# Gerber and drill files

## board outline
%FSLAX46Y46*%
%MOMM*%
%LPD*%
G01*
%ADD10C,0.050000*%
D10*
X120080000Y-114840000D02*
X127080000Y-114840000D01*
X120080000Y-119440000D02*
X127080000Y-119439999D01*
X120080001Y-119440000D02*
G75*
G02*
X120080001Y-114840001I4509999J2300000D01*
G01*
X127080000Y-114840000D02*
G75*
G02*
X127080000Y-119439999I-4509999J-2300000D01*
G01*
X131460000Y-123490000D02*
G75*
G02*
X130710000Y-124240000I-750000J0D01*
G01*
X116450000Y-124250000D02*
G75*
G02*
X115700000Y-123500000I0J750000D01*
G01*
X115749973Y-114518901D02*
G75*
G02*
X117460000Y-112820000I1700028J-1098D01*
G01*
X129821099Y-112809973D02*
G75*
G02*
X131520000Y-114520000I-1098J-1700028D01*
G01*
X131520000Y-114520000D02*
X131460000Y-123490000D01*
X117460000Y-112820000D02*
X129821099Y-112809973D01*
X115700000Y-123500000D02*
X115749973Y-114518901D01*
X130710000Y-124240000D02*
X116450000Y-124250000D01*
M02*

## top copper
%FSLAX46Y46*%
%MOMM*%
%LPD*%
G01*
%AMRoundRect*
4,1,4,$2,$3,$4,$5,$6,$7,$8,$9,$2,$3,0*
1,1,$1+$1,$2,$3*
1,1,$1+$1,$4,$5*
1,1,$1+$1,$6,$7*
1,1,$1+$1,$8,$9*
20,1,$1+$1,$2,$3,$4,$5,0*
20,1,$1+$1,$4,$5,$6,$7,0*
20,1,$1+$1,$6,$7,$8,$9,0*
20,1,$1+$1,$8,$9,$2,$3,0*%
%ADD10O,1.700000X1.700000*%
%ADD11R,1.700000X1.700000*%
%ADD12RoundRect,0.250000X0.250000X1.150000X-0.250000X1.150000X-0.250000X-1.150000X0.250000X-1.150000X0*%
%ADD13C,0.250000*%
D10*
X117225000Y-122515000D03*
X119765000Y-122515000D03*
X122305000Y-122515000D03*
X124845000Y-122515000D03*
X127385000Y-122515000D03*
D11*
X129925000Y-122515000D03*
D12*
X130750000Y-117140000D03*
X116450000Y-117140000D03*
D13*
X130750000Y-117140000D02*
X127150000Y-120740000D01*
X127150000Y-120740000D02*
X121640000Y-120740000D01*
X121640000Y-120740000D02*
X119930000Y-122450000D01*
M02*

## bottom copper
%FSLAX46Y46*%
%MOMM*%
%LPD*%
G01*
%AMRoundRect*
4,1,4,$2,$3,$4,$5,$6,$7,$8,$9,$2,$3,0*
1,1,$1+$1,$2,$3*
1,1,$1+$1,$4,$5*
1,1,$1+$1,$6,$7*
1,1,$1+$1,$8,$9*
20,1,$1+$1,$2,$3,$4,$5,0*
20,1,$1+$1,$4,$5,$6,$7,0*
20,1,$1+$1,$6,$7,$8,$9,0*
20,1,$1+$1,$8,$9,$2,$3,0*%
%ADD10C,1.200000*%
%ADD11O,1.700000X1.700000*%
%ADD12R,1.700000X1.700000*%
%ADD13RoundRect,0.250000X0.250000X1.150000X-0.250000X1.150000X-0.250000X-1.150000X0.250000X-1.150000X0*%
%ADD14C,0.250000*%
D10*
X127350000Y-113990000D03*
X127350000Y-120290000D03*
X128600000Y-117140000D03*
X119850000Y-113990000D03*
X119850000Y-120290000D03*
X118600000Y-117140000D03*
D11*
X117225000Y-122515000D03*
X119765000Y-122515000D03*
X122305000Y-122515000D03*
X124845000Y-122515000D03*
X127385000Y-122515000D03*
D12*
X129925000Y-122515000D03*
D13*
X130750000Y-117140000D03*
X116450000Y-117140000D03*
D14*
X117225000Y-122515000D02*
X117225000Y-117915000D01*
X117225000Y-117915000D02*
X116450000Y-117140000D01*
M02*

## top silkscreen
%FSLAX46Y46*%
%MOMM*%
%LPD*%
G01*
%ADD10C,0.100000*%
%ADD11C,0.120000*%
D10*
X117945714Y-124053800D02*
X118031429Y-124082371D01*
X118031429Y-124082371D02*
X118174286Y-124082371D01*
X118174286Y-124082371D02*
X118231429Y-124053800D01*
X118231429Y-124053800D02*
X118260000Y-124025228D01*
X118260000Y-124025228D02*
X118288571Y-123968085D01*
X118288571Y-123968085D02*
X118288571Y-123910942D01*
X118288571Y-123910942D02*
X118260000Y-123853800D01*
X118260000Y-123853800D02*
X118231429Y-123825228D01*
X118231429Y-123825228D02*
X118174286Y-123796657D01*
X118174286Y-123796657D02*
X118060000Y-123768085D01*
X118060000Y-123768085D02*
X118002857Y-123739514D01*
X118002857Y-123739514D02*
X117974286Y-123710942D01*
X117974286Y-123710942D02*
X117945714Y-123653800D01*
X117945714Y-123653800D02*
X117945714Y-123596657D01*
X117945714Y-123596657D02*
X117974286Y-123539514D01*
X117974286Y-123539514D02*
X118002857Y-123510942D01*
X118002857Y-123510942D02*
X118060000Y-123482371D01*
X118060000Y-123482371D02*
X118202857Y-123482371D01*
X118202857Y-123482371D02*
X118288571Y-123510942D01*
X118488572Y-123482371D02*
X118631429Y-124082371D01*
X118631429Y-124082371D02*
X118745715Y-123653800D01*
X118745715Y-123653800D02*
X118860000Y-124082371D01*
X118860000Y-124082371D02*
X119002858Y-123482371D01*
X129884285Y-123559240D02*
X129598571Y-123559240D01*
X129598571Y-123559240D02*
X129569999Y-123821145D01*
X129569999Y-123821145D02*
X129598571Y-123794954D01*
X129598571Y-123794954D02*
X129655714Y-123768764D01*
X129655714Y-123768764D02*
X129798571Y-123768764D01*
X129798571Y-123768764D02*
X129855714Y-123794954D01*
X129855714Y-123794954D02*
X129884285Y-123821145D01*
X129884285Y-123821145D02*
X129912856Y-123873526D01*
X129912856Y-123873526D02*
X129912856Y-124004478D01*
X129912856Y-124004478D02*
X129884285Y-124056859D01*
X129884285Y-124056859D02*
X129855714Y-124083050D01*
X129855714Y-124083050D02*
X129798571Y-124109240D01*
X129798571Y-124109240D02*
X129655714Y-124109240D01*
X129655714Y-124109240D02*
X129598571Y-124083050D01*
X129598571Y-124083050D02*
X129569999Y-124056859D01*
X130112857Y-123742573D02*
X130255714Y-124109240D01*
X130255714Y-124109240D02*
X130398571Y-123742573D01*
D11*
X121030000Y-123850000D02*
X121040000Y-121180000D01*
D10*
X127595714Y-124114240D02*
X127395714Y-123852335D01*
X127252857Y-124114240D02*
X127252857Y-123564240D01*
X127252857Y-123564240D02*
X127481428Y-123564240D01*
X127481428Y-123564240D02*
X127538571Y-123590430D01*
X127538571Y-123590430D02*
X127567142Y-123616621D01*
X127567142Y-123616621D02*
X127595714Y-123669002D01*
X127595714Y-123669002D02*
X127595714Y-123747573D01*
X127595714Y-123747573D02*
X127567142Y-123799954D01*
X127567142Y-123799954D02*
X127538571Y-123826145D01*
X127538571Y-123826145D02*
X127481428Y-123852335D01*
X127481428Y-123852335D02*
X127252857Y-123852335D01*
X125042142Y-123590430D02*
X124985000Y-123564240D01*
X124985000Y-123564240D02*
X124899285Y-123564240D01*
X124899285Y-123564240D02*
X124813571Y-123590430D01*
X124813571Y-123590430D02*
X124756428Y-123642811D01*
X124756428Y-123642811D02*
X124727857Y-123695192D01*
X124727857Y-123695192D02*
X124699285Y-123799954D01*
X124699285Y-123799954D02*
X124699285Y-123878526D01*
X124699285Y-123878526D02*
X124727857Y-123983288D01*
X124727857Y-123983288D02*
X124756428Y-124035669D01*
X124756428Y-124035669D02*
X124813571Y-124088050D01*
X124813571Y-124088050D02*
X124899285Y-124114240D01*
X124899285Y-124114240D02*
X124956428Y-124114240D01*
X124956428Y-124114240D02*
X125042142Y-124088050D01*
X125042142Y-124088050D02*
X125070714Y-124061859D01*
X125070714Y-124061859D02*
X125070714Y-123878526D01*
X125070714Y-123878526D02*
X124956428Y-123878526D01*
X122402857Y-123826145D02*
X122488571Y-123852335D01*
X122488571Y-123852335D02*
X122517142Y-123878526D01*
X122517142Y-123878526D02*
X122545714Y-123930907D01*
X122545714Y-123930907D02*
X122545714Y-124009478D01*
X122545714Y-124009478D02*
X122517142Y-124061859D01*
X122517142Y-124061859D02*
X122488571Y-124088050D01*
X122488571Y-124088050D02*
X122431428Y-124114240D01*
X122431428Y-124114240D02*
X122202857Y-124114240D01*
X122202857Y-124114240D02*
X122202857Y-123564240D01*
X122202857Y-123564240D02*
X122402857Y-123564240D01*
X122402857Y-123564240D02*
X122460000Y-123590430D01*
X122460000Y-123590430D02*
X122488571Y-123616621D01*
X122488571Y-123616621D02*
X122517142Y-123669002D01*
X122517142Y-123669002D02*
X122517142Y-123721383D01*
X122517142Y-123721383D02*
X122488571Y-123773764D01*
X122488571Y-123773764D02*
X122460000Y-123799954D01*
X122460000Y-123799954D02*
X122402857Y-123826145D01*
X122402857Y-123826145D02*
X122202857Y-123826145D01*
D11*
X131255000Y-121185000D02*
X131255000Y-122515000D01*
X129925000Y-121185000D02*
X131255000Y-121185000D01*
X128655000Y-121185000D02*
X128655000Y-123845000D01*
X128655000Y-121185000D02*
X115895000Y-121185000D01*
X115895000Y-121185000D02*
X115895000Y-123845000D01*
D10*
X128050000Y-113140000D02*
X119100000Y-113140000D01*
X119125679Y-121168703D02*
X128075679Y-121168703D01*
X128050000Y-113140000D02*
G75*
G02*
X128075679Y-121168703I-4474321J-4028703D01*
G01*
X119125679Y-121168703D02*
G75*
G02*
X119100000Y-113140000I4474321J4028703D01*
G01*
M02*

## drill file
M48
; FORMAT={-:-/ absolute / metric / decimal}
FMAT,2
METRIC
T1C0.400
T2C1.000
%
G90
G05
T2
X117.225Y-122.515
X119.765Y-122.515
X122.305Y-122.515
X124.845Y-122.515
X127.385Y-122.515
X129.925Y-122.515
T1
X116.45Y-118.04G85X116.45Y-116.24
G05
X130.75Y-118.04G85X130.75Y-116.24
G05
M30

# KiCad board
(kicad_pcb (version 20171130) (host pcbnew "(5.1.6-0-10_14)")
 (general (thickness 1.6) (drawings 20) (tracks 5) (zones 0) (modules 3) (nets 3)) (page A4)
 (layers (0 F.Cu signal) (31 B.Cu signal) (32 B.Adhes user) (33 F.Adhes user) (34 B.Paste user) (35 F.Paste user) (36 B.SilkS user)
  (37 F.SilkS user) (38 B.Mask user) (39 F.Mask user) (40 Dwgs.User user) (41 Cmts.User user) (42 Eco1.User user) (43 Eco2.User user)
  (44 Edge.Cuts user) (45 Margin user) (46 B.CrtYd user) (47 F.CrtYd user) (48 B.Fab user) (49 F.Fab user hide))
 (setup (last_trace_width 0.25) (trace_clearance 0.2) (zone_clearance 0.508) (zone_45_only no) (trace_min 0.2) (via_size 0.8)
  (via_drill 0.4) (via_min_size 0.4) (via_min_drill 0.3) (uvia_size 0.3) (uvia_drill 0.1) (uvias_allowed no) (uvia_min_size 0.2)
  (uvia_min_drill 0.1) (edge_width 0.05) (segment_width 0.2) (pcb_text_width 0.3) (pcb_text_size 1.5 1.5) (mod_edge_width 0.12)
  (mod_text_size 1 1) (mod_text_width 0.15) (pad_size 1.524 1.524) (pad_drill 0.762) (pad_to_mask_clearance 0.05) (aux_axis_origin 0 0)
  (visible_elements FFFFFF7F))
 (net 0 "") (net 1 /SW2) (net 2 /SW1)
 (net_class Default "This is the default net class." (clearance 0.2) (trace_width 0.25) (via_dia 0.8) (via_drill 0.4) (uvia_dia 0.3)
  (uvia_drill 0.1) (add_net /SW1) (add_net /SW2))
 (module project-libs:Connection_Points (layer B.Cu) (at 123.6 117.14)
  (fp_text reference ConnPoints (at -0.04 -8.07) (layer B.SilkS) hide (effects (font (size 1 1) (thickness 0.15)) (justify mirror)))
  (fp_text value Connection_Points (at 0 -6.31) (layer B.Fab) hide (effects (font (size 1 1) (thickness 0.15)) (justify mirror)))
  (pad "" smd circle (at 3.75 -3.15) (size 1.2 1.2) (layers B.Cu B.Paste B.Mask))
  (pad "" smd circle (at 3.75 3.15) (size 1.2 1.2) (layers B.Cu B.Paste B.Mask))
  (pad "" smd circle (at 5 0) (size 1.2 1.2) (layers B.Cu B.Paste B.Mask))
  (pad "" smd circle (at -3.75 -3.15) (size 1.2 1.2) (layers B.Cu B.Paste B.Mask))
  (pad "" smd circle (at -3.75 3.15) (size 1.2 1.2) (layers B.Cu B.Paste B.Mask))
  (pad "" smd circle (at -5 0) (size 1.2 1.2) (layers B.Cu B.Paste B.Mask)))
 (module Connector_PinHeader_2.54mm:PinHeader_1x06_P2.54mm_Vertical (layer F.Cu) (at 129.925 122.515 270)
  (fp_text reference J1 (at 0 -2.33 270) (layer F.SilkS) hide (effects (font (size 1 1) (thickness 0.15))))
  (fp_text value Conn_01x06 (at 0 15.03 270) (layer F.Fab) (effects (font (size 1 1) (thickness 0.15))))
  (fp_line (start -1.33 -1.33) (end 0 -1.33) (layer F.SilkS) (width 0.12))
  (fp_line (start -1.33 0) (end -1.33 -1.33) (layer F.SilkS) (width 0.12))
  (fp_line (start -1.33 1.27) (end 1.33 1.27) (layer F.SilkS) (width 0.12))
  (fp_line (start -1.33 1.27) (end -1.33 14.03) (layer F.SilkS) (width 0.12))
  (fp_line (start -1.33 14.03) (end 1.33 14.03) (layer F.SilkS) (width 0.12))
  (pad 6 thru_hole oval (at 0 12.7 270) (size 1.7 1.7) (drill 1) (layers *.Cu *.Mask) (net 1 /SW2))
  (pad 5 thru_hole oval (at 0 10.16 270) (size 1.7 1.7) (drill 1) (layers *.Cu *.Mask) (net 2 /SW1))
  (pad 4 thru_hole oval (at 0 7.62 270) (size 1.7 1.7) (drill 1) (layers *.Cu *.Mask))
  (pad 3 thru_hole oval (at 0 5.08 270) (size 1.7 1.7) (drill 1) (layers *.Cu *.Mask))
  (pad 2 thru_hole oval (at 0 2.54 270) (size 1.7 1.7) (drill 1) (layers *.Cu *.Mask))
  (pad 1 thru_hole rect (at 0 0 270) (size 1.7 1.7) (drill 1) (layers *.Cu *.Mask)))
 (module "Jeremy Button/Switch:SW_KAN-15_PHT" (layer F.Cu) (at 123.6 117.14 180)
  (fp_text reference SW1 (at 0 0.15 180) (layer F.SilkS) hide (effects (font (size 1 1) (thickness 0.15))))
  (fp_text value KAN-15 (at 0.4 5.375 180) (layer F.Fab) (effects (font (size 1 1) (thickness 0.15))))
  (fp_line (start -4.45 4) (end 4.5 4) (layer F.SilkS) (width 0.1))
  (fp_line (start 4.474321 -4.028703) (end -4.475679 -4.028703) (layer F.SilkS) (width 0.1))
  (fp_arc (start 0.024321 -0.028703) (end -4.475679 -4.028703) (angle -83.63358372) (layer F.SilkS) (width 0.1))
  (fp_arc (start 0 0) (end 4.5 4) (angle -83.63358372) (layer F.SilkS) (width 0.1))
  (pad 1 thru_hole roundrect (at -7.15 0 180) (size 1 2.8) (drill oval 0.4 2.2) (layers *.Cu *.Mask) (roundrect_rratio 0.25) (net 2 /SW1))
  (pad 2 thru_hole roundrect (at 7.15 0 180) (size 1 2.8) (drill oval 0.4 2.2) (layers *.Cu *.Mask) (roundrect_rratio 0.25) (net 1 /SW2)))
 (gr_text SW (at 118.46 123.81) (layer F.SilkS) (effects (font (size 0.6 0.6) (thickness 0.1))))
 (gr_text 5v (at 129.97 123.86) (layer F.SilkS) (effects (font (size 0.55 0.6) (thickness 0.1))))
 (gr_line (start 121.03 123.85) (end 121.04 121.18) (layer F.SilkS) (width 0.12))
 (gr_line (start 120.08 114.84) (end 127.08 114.84) (layer Edge.Cuts) (width 0.05))
 (gr_line (start 120.08 119.44) (end 127.08 119.439999) (layer Edge.Cuts) (width 0.05))
 (gr_arc (start 124.59 117.14) (end 120.080001 114.840001) (angle -54.04114679) (layer Edge.Cuts) (width 0.05))
 (gr_arc (start 122.570001 117.14) (end 127.08 119.439999) (angle -54.04114679) (layer Edge.Cuts) (width 0.05))
 (gr_arc (start 130.71 123.49) (end 130.71 124.24) (angle -90) (layer Edge.Cuts) (width 0.05))
 (gr_arc (start 116.45 123.5) (end 115.7 123.5) (angle -90) (layer Edge.Cuts) (width 0.05))
 (gr_arc (start 117.450001 114.519999) (end 117.46 112.82) (angle -90.3) (layer Edge.Cuts) (width 0.05))
 (gr_arc (start 129.820001 114.510001) (end 131.52 114.52) (angle -90.3) (layer Edge.Cuts) (width 0.05))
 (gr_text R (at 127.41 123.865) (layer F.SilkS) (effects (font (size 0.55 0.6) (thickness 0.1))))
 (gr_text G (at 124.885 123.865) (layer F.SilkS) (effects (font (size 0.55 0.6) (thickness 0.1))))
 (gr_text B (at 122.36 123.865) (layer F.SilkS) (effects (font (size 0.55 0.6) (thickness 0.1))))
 (gr_line (start 131.52 114.52) (end 131.46 123.49) (layer Edge.Cuts) (width 0.05))
 (gr_line (start 117.46 112.82) (end 129.821099 112.809973) (layer Edge.Cuts) (width 0.05))
 (gr_line (start 115.7 123.5) (end 115.749973 114.518901) (layer Edge.Cuts) (width 0.05))
 (gr_line (start 130.71 124.24) (end 116.45 124.25) (layer Edge.Cuts) (width 0.05))
 (segment (start 130.75 117.14) (end 127.15 120.74) (width 0.25) (layer F.Cu) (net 2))
 (segment (start 127.15 120.74) (end 121.64 120.74) (width 0.25) (layer F.Cu) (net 2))
 (segment (start 121.64 120.74) (end 119.93 122.45) (width 0.25) (layer F.Cu) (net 2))
 (segment (start 117.225 122.515) (end 117.225 117.915) (width 0.25) (layer B.Cu) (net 1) (status 1000000))
 (segment (start 117.225 117.915) (end 116.45 117.14) (width 0.25) (layer B.Cu) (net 1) (status 1000000)))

